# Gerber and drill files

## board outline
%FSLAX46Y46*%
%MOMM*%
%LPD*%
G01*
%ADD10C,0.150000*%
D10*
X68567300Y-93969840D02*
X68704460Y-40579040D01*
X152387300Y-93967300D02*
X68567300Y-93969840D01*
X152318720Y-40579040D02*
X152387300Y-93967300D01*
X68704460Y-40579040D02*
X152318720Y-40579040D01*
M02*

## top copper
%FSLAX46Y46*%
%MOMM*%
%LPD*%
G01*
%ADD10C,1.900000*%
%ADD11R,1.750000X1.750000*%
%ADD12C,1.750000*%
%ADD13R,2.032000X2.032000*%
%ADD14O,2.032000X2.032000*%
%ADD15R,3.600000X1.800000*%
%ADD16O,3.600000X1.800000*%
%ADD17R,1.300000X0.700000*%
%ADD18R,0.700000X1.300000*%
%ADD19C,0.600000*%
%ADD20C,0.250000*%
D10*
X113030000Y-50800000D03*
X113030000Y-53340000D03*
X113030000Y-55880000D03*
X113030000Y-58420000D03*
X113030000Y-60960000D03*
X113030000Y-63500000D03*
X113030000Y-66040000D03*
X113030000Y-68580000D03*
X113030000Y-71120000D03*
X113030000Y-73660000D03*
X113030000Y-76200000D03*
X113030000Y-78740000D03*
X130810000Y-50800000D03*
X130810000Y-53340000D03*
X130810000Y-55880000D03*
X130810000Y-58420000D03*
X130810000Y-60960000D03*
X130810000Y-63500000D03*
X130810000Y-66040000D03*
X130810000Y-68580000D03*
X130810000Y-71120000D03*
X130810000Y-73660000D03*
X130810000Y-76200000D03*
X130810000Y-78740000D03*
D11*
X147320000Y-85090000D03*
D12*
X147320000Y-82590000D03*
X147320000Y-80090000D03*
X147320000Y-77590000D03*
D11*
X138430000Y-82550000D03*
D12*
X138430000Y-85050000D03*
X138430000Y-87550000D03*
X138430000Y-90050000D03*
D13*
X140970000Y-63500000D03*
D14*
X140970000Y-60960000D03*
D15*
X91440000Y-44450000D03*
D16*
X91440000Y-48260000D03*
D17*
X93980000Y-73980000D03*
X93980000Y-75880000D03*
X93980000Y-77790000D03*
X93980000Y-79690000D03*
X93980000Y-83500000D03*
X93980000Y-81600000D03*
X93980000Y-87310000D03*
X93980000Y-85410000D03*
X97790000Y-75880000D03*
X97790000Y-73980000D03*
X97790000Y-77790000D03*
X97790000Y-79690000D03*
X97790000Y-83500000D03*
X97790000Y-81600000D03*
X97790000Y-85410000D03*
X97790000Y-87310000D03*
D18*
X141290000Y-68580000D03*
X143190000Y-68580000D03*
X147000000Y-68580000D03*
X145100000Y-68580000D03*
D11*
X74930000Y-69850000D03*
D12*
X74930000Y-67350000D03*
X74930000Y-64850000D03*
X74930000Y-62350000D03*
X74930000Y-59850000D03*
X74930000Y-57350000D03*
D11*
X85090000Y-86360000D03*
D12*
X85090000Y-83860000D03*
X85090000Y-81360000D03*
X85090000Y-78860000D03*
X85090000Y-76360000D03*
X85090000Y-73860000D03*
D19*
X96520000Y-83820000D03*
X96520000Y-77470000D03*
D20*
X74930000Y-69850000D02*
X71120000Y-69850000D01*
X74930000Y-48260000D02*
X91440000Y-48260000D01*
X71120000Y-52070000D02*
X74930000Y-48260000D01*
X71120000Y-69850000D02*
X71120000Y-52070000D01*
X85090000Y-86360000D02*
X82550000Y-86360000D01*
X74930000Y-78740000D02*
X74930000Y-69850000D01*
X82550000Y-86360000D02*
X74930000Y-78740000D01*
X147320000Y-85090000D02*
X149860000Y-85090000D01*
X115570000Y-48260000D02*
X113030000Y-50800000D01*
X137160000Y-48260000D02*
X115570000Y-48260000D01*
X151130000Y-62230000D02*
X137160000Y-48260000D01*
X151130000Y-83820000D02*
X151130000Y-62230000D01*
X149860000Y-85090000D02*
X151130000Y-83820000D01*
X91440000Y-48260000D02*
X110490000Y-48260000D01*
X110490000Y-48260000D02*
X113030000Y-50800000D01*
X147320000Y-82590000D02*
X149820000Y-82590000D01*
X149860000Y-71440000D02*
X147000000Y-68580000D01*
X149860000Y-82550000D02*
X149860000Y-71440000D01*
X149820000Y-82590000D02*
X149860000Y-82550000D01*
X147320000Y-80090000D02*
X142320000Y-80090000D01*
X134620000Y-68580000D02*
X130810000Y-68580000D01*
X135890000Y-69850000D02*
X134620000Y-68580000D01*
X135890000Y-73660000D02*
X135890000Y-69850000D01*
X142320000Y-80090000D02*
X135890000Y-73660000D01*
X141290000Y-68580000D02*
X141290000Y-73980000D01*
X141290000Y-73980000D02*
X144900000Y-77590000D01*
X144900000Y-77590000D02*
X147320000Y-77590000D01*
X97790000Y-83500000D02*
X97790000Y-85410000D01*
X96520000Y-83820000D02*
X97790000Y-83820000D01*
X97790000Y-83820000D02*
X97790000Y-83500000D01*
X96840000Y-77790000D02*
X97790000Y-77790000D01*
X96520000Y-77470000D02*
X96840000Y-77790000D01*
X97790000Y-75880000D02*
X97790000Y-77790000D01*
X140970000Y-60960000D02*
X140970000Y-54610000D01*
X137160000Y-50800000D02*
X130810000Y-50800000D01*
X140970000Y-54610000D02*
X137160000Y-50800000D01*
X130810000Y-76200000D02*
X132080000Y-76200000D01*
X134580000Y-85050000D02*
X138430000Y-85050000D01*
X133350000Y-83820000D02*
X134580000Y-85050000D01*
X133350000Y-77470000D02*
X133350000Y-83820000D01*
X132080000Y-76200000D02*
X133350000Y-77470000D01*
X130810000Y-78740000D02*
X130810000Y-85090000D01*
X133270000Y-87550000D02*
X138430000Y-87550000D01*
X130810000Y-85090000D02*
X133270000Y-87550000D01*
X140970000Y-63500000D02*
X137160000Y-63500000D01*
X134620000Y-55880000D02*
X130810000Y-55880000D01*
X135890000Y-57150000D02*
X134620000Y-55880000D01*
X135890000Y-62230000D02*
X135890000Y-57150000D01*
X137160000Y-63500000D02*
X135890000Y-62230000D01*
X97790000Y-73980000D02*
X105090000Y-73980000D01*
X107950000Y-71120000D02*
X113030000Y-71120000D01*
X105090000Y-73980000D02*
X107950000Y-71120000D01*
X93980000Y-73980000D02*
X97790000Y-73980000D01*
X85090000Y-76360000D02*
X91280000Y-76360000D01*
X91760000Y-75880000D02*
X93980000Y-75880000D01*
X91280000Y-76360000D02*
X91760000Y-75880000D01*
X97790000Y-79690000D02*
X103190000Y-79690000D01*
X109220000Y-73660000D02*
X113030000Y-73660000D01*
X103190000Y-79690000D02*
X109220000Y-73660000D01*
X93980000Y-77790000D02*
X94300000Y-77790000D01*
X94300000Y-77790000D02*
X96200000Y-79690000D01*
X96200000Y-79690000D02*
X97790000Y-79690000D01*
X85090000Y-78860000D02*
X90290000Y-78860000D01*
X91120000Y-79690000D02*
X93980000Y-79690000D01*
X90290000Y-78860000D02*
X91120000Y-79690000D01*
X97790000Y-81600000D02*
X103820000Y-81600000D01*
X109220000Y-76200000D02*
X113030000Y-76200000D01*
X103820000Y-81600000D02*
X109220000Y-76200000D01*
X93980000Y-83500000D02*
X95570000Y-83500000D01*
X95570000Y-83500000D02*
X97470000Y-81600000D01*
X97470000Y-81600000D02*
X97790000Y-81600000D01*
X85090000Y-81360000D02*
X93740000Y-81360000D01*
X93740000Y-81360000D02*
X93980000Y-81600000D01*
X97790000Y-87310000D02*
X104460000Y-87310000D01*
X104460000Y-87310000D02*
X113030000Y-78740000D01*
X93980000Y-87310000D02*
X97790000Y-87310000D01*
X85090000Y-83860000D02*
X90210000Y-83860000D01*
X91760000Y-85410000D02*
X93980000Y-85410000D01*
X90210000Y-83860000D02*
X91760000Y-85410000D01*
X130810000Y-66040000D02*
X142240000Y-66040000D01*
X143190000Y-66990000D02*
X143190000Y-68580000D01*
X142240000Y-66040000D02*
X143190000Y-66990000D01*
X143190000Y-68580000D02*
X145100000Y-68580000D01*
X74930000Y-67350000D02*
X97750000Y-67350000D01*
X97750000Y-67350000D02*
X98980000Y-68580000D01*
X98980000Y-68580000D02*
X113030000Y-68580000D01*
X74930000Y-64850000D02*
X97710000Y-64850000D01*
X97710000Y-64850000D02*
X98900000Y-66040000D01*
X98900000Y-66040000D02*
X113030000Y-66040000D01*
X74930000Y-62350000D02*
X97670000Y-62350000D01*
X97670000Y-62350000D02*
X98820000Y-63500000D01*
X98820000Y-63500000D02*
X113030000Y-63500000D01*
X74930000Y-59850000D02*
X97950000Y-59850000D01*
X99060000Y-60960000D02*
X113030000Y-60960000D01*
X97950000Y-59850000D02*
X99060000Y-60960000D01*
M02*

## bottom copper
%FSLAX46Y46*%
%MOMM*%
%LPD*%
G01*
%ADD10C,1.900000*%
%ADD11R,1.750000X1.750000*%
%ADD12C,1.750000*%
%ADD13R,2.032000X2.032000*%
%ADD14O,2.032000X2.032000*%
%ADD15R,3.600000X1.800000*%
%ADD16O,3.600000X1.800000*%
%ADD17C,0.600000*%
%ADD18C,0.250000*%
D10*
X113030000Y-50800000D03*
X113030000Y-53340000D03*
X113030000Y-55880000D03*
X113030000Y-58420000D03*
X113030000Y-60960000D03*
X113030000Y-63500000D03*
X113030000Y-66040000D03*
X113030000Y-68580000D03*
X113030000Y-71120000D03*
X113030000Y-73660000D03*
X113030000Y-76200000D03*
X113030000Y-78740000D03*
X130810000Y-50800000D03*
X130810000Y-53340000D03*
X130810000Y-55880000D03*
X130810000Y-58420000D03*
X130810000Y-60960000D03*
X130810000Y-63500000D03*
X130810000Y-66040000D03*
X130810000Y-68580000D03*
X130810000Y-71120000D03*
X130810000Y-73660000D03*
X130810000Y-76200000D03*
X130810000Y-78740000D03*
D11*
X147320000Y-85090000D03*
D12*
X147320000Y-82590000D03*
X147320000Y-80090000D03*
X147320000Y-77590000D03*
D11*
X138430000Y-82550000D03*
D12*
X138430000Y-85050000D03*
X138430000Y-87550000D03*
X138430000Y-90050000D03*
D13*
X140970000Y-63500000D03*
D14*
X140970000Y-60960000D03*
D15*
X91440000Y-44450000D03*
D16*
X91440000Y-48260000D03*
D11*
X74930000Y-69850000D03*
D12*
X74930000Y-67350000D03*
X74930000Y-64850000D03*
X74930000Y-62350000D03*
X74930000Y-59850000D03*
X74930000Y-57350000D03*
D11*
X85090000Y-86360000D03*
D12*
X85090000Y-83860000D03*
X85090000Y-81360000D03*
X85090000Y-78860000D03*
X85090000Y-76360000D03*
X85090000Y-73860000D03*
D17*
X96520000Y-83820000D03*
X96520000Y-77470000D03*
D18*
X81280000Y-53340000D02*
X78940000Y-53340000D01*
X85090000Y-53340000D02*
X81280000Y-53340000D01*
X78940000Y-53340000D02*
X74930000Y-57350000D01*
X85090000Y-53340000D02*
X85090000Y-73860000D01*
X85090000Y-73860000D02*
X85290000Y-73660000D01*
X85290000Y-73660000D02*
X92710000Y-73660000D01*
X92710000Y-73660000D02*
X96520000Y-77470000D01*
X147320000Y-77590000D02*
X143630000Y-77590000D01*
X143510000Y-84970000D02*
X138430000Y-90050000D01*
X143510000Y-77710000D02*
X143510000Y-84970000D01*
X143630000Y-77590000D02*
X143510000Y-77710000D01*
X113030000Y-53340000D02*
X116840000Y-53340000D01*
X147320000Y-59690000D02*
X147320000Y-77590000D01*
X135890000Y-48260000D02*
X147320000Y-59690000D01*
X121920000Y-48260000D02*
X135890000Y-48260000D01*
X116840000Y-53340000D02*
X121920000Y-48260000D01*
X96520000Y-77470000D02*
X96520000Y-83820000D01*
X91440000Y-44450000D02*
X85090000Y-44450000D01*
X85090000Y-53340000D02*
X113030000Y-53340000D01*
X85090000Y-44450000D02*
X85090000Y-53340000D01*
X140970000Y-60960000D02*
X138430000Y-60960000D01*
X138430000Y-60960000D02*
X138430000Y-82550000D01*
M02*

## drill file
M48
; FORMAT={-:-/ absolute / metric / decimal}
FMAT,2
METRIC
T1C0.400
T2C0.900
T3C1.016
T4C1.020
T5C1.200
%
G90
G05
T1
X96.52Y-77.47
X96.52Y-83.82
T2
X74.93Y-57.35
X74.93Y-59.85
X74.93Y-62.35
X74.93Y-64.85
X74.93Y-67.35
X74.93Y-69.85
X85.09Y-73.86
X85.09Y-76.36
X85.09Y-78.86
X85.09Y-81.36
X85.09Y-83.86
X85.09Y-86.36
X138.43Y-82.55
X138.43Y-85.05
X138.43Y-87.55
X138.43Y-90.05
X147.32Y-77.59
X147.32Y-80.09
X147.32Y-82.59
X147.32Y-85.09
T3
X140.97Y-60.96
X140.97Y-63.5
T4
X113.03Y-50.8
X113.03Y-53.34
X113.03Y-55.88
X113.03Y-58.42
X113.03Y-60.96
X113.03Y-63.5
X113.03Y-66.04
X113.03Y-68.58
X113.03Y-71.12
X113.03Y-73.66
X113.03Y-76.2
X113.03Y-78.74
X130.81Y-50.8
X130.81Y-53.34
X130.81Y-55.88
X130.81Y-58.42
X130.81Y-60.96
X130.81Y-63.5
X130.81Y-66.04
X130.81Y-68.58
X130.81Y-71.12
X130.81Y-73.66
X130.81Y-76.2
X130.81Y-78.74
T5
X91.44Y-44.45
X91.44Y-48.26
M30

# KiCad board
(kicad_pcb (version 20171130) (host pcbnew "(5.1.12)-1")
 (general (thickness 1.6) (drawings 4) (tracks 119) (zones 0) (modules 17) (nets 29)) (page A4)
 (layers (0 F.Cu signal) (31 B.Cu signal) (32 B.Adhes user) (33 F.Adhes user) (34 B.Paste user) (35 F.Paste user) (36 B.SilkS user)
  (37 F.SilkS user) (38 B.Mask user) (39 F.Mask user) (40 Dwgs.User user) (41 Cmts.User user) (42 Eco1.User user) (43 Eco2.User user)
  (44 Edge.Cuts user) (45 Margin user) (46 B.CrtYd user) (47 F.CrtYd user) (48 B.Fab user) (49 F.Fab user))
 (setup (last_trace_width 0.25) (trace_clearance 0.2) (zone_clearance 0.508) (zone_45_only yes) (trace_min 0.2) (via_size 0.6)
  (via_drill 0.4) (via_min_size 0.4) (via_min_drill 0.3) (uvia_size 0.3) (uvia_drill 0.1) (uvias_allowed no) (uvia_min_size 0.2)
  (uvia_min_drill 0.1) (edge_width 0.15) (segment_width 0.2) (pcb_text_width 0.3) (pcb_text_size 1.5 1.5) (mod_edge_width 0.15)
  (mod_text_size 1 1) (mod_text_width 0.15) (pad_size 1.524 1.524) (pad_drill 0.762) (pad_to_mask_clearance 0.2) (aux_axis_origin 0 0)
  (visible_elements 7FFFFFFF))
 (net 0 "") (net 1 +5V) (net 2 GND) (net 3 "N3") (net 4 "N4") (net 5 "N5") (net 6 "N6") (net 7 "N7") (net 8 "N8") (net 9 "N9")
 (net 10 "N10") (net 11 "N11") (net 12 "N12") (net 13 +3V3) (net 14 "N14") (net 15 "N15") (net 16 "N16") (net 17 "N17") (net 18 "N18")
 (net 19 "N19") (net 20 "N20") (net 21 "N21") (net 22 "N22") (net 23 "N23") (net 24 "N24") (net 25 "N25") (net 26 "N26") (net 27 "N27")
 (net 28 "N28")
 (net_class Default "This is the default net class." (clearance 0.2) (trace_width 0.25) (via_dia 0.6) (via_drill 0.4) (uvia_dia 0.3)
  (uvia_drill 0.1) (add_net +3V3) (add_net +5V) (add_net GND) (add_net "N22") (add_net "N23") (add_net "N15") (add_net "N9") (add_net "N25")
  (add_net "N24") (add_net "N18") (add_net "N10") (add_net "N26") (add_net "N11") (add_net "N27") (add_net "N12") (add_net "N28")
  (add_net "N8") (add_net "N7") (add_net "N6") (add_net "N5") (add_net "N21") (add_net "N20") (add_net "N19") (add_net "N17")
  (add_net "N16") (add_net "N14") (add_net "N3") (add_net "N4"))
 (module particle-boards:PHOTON (layer F.Cu) (at 121.92 66.04)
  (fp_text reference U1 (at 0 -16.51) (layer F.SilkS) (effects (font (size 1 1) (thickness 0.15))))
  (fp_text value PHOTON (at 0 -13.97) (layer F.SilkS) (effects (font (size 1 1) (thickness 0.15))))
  (pad 1 thru_hole circle (at -8.89 -15.24) (size 1.9 1.9) (drill 1.02) (layers *.Cu *.Mask F.SilkS) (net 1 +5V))
  (pad 2 thru_hole circle (at -8.89 -12.7) (size 1.9 1.9) (drill 1.02) (layers *.Cu *.Mask F.SilkS) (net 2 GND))
  (pad 3 thru_hole circle (at -8.89 -10.16) (size 1.9 1.9) (drill 1.02) (layers *.Cu *.Mask F.SilkS) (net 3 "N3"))
  (pad 4 thru_hole circle (at -8.89 -7.62) (size 1.9 1.9) (drill 1.02) (layers *.Cu *.Mask F.SilkS) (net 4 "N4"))
  (pad 5 thru_hole circle (at -8.89 -5.08) (size 1.9 1.9) (drill 1.02) (layers *.Cu *.Mask F.SilkS) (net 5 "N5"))
  (pad 6 thru_hole circle (at -8.89 -2.54) (size 1.9 1.9) (drill 1.02) (layers *.Cu *.Mask F.SilkS) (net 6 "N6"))
  (pad 7 thru_hole circle (at -8.89 0) (size 1.9 1.9) (drill 1.02) (layers *.Cu *.Mask F.SilkS) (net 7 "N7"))
  (pad 8 thru_hole circle (at -8.89 2.54) (size 1.9 1.9) (drill 1.02) (layers *.Cu *.Mask F.SilkS) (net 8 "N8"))
  (pad 9 thru_hole circle (at -8.89 5.08) (size 1.9 1.9) (drill 1.02) (layers *.Cu *.Mask F.SilkS) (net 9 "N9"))
  (pad 10 thru_hole circle (at -8.89 7.62) (size 1.9 1.9) (drill 1.02) (layers *.Cu *.Mask F.SilkS) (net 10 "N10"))
  (pad 11 thru_hole circle (at -8.89 10.16) (size 1.9 1.9) (drill 1.02) (layers *.Cu *.Mask F.SilkS) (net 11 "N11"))
  (pad 12 thru_hole circle (at -8.89 12.7) (size 1.9 1.9) (drill 1.02) (layers *.Cu *.Mask F.SilkS) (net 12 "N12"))
  (pad 24 thru_hole circle (at 8.89 -15.24) (size 1.9 1.9) (drill 1.02) (layers *.Cu *.Mask F.SilkS) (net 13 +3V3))
  (pad 23 thru_hole circle (at 8.89 -12.7) (size 1.9 1.9) (drill 1.02) (layers *.Cu *.Mask F.SilkS) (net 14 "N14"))
  (pad 22 thru_hole circle (at 8.89 -10.16) (size 1.9 1.9) (drill 1.02) (layers *.Cu *.Mask F.SilkS) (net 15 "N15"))
  (pad 21 thru_hole circle (at 8.89 -7.62) (size 1.9 1.9) (drill 1.02) (layers *.Cu *.Mask F.SilkS))
  (pad 20 thru_hole circle (at 8.89 -5.08) (size 1.9 1.9) (drill 1.02) (layers *.Cu *.Mask F.SilkS) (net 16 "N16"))
  (pad 19 thru_hole circle (at 8.89 -2.54) (size 1.9 1.9) (drill 1.02) (layers *.Cu *.Mask F.SilkS) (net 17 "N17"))
  (pad 18 thru_hole circle (at 8.89 0) (size 1.9 1.9) (drill 1.02) (layers *.Cu *.Mask F.SilkS) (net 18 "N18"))
  (pad 17 thru_hole circle (at 8.89 2.54) (size 1.9 1.9) (drill 1.02) (layers *.Cu *.Mask F.SilkS) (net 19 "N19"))
  (pad 16 thru_hole circle (at 8.89 5.08) (size 1.9 1.9) (drill 1.02) (layers *.Cu *.Mask F.SilkS) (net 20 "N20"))
  (pad 15 thru_hole circle (at 8.89 7.62) (size 1.9 1.9) (drill 1.02) (layers *.Cu *.Mask F.SilkS) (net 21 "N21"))
  (pad 14 thru_hole circle (at 8.89 10.16) (size 1.9 1.9) (drill 1.02) (layers *.Cu *.Mask F.SilkS) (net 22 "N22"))
  (pad 13 thru_hole circle (at 8.89 12.7) (size 1.9 1.9) (drill 1.02) (layers *.Cu *.Mask F.SilkS) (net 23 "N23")))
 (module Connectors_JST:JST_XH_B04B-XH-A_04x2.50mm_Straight (layer F.Cu) (at 147.32 85.09 90)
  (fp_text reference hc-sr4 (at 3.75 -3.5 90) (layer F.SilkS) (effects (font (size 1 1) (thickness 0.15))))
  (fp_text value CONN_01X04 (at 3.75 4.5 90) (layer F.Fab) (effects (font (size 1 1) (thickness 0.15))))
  (pad 1 thru_hole rect (at 0 0 90) (size 1.75 1.75) (drill 0.9) (layers *.Cu *.Mask) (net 1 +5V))
  (pad 2 thru_hole circle (at 2.5 0 90) (size 1.75 1.75) (drill 0.9) (layers *.Cu *.Mask) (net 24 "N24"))
  (pad 3 thru_hole circle (at 5 0 90) (size 1.75 1.75) (drill 0.9) (layers *.Cu *.Mask) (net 19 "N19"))
  (pad 4 thru_hole circle (at 7.5 0 90) (size 1.75 1.75) (drill 0.9) (layers *.Cu *.Mask) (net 2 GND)))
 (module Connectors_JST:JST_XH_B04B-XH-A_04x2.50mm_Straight (layer F.Cu) (at 138.43 82.55 270)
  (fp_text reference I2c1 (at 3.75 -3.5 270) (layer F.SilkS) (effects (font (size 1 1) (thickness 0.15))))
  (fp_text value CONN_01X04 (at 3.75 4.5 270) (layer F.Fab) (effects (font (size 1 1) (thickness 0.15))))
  (pad 1 thru_hole rect (at 0 0 270) (size 1.75 1.75) (drill 0.9) (layers *.Cu *.Mask) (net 13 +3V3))
  (pad 2 thru_hole circle (at 2.5 0 270) (size 1.75 1.75) (drill 0.9) (layers *.Cu *.Mask) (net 22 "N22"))
  (pad 3 thru_hole circle (at 5 0 270) (size 1.75 1.75) (drill 0.9) (layers *.Cu *.Mask) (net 23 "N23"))
  (pad 4 thru_hole circle (at 7.5 0 270) (size 1.75 1.75) (drill 0.9) (layers *.Cu *.Mask) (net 2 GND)))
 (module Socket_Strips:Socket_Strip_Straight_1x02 (layer F.Cu) (at 140.97 63.5 90)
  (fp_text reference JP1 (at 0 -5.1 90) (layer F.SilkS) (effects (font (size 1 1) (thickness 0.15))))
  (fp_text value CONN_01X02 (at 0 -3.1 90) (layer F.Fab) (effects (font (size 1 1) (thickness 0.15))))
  (pad 1 thru_hole rect (at 0 0 90) (size 2.032 2.032) (drill 1.016) (layers *.Cu *.Mask F.SilkS) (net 15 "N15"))
  (pad 2 thru_hole oval (at 2.54 0 90) (size 2.032 2.032) (drill 1.016) (layers *.Cu *.Mask F.SilkS) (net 13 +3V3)))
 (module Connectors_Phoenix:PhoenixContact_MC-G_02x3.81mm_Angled (layer F.Cu) (at 91.44 44.45 270)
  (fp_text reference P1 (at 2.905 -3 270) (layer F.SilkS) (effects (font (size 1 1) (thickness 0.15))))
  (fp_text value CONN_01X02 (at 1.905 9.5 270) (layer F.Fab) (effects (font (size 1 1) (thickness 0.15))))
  (pad 1 thru_hole rect (at 0 0 270) (size 1.8 3.6) (drill 1.2) (layers *.Cu *.Mask) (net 2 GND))
  (pad 2 thru_hole oval (at 3.81 0 270) (size 1.8 3.6) (drill 1.2) (layers *.Cu *.Mask) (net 1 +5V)))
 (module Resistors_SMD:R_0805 (layer F.Cu) (at 93.98 74.93 270)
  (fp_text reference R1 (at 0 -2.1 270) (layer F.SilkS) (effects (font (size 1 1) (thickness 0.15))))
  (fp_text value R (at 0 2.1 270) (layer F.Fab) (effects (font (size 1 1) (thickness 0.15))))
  (pad 1 smd rect (at -0.95 0 270) (size 0.7 1.3) (layers F.Cu F.Paste F.Mask) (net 9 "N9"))
  (pad 2 smd rect (at 0.95 0 270) (size 0.7 1.3) (layers F.Cu F.Paste F.Mask) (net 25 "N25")))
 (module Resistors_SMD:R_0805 (layer F.Cu) (at 93.98 78.74 270)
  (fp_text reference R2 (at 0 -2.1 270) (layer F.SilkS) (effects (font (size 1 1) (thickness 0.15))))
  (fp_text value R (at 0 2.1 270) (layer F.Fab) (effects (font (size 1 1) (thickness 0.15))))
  (pad 1 smd rect (at -0.95 0 270) (size 0.7 1.3) (layers F.Cu F.Paste F.Mask) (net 10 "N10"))
  (pad 2 smd rect (at 0.95 0 270) (size 0.7 1.3) (layers F.Cu F.Paste F.Mask) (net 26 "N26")))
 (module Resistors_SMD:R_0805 (layer F.Cu) (at 93.98 82.55 90)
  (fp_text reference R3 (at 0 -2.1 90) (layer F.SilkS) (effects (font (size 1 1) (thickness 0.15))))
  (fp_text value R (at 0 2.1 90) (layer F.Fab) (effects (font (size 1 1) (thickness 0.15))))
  (pad 1 smd rect (at -0.95 0 90) (size 0.7 1.3) (layers F.Cu F.Paste F.Mask) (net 11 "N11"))
  (pad 2 smd rect (at 0.95 0 90) (size 0.7 1.3) (layers F.Cu F.Paste F.Mask) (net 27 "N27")))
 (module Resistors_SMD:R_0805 (layer F.Cu) (at 93.98 86.36 90)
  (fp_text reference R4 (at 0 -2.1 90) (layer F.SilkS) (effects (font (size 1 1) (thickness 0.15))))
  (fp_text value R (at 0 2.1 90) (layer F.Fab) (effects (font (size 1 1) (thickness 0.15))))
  (pad 1 smd rect (at -0.95 0 90) (size 0.7 1.3) (layers F.Cu F.Paste F.Mask) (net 12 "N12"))
  (pad 2 smd rect (at 0.95 0 90) (size 0.7 1.3) (layers F.Cu F.Paste F.Mask) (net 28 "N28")))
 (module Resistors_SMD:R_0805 (layer F.Cu) (at 97.79 74.93 90)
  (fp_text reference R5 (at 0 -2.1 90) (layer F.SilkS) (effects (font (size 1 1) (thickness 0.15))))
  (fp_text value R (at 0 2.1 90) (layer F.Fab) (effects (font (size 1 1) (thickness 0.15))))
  (pad 1 smd rect (at -0.95 0 90) (size 0.7 1.3) (layers F.Cu F.Paste F.Mask) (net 2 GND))
  (pad 2 smd rect (at 0.95 0 90) (size 0.7 1.3) (layers F.Cu F.Paste F.Mask) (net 9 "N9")))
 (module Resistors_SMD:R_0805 (layer F.Cu) (at 97.79 78.74 270)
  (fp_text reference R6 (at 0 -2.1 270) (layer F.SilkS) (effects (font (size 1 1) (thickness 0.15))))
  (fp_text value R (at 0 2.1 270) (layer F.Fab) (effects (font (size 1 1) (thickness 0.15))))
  (pad 1 smd rect (at -0.95 0 270) (size 0.7 1.3) (layers F.Cu F.Paste F.Mask) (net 2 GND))
  (pad 2 smd rect (at 0.95 0 270) (size 0.7 1.3) (layers F.Cu F.Paste F.Mask) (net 10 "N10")))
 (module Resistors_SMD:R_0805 (layer F.Cu) (at 97.79 82.55 90)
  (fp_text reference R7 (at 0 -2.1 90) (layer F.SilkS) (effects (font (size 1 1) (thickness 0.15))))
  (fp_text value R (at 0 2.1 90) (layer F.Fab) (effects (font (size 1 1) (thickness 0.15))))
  (pad 1 smd rect (at -0.95 0 90) (size 0.7 1.3) (layers F.Cu F.Paste F.Mask) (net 2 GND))
  (pad 2 smd rect (at 0.95 0 90) (size 0.7 1.3) (layers F.Cu F.Paste F.Mask) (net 11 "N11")))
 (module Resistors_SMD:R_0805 (layer F.Cu) (at 97.79 86.36 270)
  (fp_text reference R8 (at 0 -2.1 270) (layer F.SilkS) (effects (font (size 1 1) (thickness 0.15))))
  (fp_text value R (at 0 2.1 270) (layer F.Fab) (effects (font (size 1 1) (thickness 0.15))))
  (pad 1 smd rect (at -0.95 0 270) (size 0.7 1.3) (layers F.Cu F.Paste F.Mask) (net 2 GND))
  (pad 2 smd rect (at 0.95 0 270) (size 0.7 1.3) (layers F.Cu F.Paste F.Mask) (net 12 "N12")))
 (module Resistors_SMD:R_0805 (layer F.Cu) (at 142.24 68.58)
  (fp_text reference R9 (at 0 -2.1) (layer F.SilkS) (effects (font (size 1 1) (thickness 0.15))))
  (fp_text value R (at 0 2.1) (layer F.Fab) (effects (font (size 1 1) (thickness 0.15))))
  (pad 1 smd rect (at -0.95 0) (size 0.7 1.3) (layers F.Cu F.Paste F.Mask) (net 2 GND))
  (pad 2 smd rect (at 0.95 0) (size 0.7 1.3) (layers F.Cu F.Paste F.Mask) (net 18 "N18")))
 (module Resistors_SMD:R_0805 (layer F.Cu) (at 146.05 68.58 180)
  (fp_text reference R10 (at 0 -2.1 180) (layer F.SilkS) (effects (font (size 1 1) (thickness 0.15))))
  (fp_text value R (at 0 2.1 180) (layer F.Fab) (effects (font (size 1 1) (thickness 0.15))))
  (pad 1 smd rect (at -0.95 0 180) (size 0.7 1.3) (layers F.Cu F.Paste F.Mask) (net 24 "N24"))
  (pad 2 smd rect (at 0.95 0 180) (size 0.7 1.3) (layers F.Cu F.Paste F.Mask) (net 18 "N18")))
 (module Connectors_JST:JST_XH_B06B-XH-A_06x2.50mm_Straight (layer F.Cu) (at 74.93 69.85 90)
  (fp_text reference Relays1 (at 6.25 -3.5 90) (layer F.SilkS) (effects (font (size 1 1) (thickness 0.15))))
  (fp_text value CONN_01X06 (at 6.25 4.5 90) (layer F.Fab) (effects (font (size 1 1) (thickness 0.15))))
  (pad 1 thru_hole rect (at 0 0 90) (size 1.75 1.75) (drill 0.9) (layers *.Cu *.Mask) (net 1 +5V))
  (pad 2 thru_hole circle (at 2.5 0 90) (size 1.75 1.75) (drill 0.9) (layers *.Cu *.Mask) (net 8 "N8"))
  (pad 3 thru_hole circle (at 5 0 90) (size 1.75 1.75) (drill 0.9) (layers *.Cu *.Mask) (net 7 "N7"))
  (pad 4 thru_hole circle (at 7.5 0 90) (size 1.75 1.75) (drill 0.9) (layers *.Cu *.Mask) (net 6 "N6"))
  (pad 5 thru_hole circle (at 10 0 90) (size 1.75 1.75) (drill 0.9) (layers *.Cu *.Mask) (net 5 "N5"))
  (pad 6 thru_hole circle (at 12.5 0 90) (size 1.75 1.75) (drill 0.9) (layers *.Cu *.Mask) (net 2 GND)))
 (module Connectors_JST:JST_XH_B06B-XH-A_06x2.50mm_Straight (layer F.Cu) (at 85.09 86.36 90)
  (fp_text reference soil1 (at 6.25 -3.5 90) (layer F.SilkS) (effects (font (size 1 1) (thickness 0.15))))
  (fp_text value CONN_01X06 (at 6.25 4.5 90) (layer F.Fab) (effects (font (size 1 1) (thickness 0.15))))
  (pad 1 thru_hole rect (at 0 0 90) (size 1.75 1.75) (drill 0.9) (layers *.Cu *.Mask) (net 1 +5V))
  (pad 2 thru_hole circle (at 2.5 0 90) (size 1.75 1.75) (drill 0.9) (layers *.Cu *.Mask) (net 28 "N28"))
  (pad 3 thru_hole circle (at 5 0 90) (size 1.75 1.75) (drill 0.9) (layers *.Cu *.Mask) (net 27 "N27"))
  (pad 4 thru_hole circle (at 7.5 0 90) (size 1.75 1.75) (drill 0.9) (layers *.Cu *.Mask) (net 26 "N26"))
  (pad 5 thru_hole circle (at 10 0 90) (size 1.75 1.75) (drill 0.9) (layers *.Cu *.Mask) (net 25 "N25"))
  (pad 6 thru_hole circle (at 12.5 0 90) (size 1.75 1.75) (drill 0.9) (layers *.Cu *.Mask) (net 2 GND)))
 (gr_line (start 68.5673 93.96984) (end 68.70446 40.57904) (layer Edge.Cuts) (width 0.15))
 (gr_line (start 152.3873 93.9673) (end 68.5673 93.96984) (layer Edge.Cuts) (width 0.15))
 (gr_line (start 152.31872 40.57904) (end 152.3873 93.9673) (layer Edge.Cuts) (width 0.15))
 (gr_line (start 68.70446 40.57904) (end 152.31872 40.57904) (layer Edge.Cuts) (width 0.15))
 (segment (start 74.93 69.85) (end 71.12 69.85) (width 0.25) (layer F.Cu) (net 1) (status 400000))
 (segment (start 74.93 48.26) (end 91.44 48.26) (width 0.25) (layer F.Cu) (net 1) (status 800000))
 (segment (start 71.12 52.07) (end 74.93 48.26) (width 0.25) (layer F.Cu) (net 1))
 (segment (start 71.12 69.85) (end 71.12 52.07) (width 0.25) (layer F.Cu) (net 1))
 (segment (start 85.09 86.36) (end 82.55 86.36) (width 0.25) (layer F.Cu) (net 1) (status 400000))
 (segment (start 74.93 78.74) (end 74.93 69.85) (width 0.25) (layer F.Cu) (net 1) (status 800000))
 (segment (start 82.55 86.36) (end 74.93 78.74) (width 0.25) (layer F.Cu) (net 1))
 (segment (start 147.32 85.09) (end 149.86 85.09) (width 0.25) (layer F.Cu) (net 1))
 (segment (start 115.57 48.26) (end 113.03 50.8) (width 0.25) (layer F.Cu) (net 1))
 (segment (start 137.16 48.26) (end 115.57 48.26) (width 0.25) (layer F.Cu) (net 1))
 (segment (start 151.13 62.23) (end 137.16 48.26) (width 0.25) (layer F.Cu) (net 1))
 (segment (start 151.13 83.82) (end 151.13 62.23) (width 0.25) (layer F.Cu) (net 1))
 (segment (start 149.86 85.09) (end 151.13 83.82) (width 0.25) (layer F.Cu) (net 1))
 (segment (start 91.44 48.26) (end 110.49 48.26) (width 0.25) (layer F.Cu) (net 1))
 (segment (start 110.49 48.26) (end 113.03 50.8) (width 0.25) (layer F.Cu) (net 1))
 (segment (start 147.32 82.59) (end 149.82 82.59) (width 0.25) (layer F.Cu) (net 24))
 (segment (start 149.86 71.44) (end 147 68.58) (width 0.25) (layer F.Cu) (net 24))
 (segment (start 149.86 82.55) (end 149.86 71.44) (width 0.25) (layer F.Cu) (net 24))
 (segment (start 149.82 82.59) (end 149.86 82.55) (width 0.25) (layer F.Cu) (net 24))
 (segment (start 147.32 80.09) (end 142.32 80.09) (width 0.25) (layer F.Cu) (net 19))
 (segment (start 134.62 68.58) (end 130.81 68.58) (width 0.25) (layer F.Cu) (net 19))
 (segment (start 135.89 69.85) (end 134.62 68.58) (width 0.25) (layer F.Cu) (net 19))
 (segment (start 135.89 73.66) (end 135.89 69.85) (width 0.25) (layer F.Cu) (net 19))
 (segment (start 142.32 80.09) (end 135.89 73.66) (width 0.25) (layer F.Cu) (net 19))
 (segment (start 81.28 53.34) (end 78.94 53.34) (width 0.25) (layer B.Cu) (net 2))
 (segment (start 85.09 53.34) (end 81.28 53.34) (width 0.25) (layer B.Cu) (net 2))
 (segment (start 78.94 53.34) (end 74.93 57.35) (width 0.25) (layer B.Cu) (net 2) (status 800000))
 (segment (start 85.09 53.34) (end 85.09 73.86) (width 0.25) (layer B.Cu) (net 2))
 (segment (start 85.09 73.86) (end 85.29 73.66) (width 0.25) (layer B.Cu) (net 2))
 (segment (start 85.29 73.66) (end 92.71 73.66) (width 0.25) (layer B.Cu) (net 2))
 (segment (start 92.71 73.66) (end 96.52 77.47) (width 0.25) (layer B.Cu) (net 2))
 (segment (start 147.32 77.59) (end 143.63 77.59) (width 0.25) (layer B.Cu) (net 2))
 (segment (start 143.51 84.97) (end 138.43 90.05) (width 0.25) (layer B.Cu) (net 2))
 (segment (start 143.51 77.71) (end 143.51 84.97) (width 0.25) (layer B.Cu) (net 2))
 (segment (start 143.63 77.59) (end 143.51 77.71) (width 0.25) (layer B.Cu) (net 2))
 (segment (start 113.03 53.34) (end 116.84 53.34) (width 0.25) (layer B.Cu) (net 2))
 (segment (start 147.32 59.69) (end 147.32 77.59) (width 0.25) (layer B.Cu) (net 2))
 (segment (start 135.89 48.26) (end 147.32 59.69) (width 0.25) (layer B.Cu) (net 2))
 (segment (start 121.92 48.26) (end 135.89 48.26) (width 0.25) (layer B.Cu) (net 2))
 (segment (start 116.84 53.34) (end 121.92 48.26) (width 0.25) (layer B.Cu) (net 2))
 (segment (start 141.29 68.58) (end 141.29 73.98) (width 0.25) (layer F.Cu) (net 2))
 (segment (start 141.29 73.98) (end 144.9 77.59) (width 0.25) (layer F.Cu) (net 2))
 (segment (start 144.9 77.59) (end 147.32 77.59) (width 0.25) (layer F.Cu) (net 2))
 (segment (start 97.79 83.5) (end 97.79 85.41) (width 0.25) (layer F.Cu) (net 2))
 (segment (start 96.52 77.47) (end 96.52 83.82) (width 0.25) (layer B.Cu) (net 2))
 (segment (start 96.52 83.82) (end 97.79 83.82) (width 0.25) (layer F.Cu) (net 2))
 (via (at 96.52 83.82) (size 0.6) (drill 0.4) (layers F.Cu B.Cu) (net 2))
 (segment (start 97.79 83.82) (end 97.79 83.5) (width 0.25) (layer F.Cu) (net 2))
 (segment (start 96.84 77.79) (end 97.79 77.79) (width 0.25) (layer F.Cu) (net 2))
 (segment (start 96.52 77.47) (end 96.84 77.79) (width 0.25) (layer F.Cu) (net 2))
 (via (at 96.52 77.47) (size 0.6) (drill 0.4) (layers F.Cu B.Cu) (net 2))
 (segment (start 97.79 75.88) (end 97.79 77.79) (width 0.25) (layer F.Cu) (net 2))
 (segment (start 91.44 44.45) (end 85.09 44.45) (width 0.25) (layer B.Cu) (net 2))
 (segment (start 85.09 53.34) (end 113.03 53.34) (width 0.25) (layer B.Cu) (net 2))
 (segment (start 85.09 44.45) (end 85.09 53.34) (width 0.25) (layer B.Cu) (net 2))
 (segment (start 140.97 60.96) (end 138.43 60.96) (width 0.25) (layer B.Cu) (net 13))
 (segment (start 138.43 60.96) (end 138.43 82.55) (width 0.25) (layer B.Cu) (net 13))
 (segment (start 140.97 60.96) (end 140.97 54.61) (width 0.25) (layer F.Cu) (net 13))
 (segment (start 137.16 50.8) (end 130.81 50.8) (width 0.25) (layer F.Cu) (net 13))
 (segment (start 140.97 54.61) (end 137.16 50.8) (width 0.25) (layer F.Cu) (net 13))
 (segment (start 130.81 76.2) (end 132.08 76.2) (width 0.25) (layer F.Cu) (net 22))
 (segment (start 134.58 85.05) (end 138.43 85.05) (width 0.25) (layer F.Cu) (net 22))
 (segment (start 133.35 83.82) (end 134.58 85.05) (width 0.25) (layer F.Cu) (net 22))
 (segment (start 133.35 77.47) (end 133.35 83.82) (width 0.25) (layer F.Cu) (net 22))
 (segment (start 132.08 76.2) (end 133.35 77.47) (width 0.25) (layer F.Cu) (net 22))
 (segment (start 130.81 78.74) (end 130.81 85.09) (width 0.25) (layer F.Cu) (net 23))
 (segment (start 133.27 87.55) (end 138.43 87.55) (width 0.25) (layer F.Cu) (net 23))
 (segment (start 130.81 85.09) (end 133.27 87.55) (width 0.25) (layer F.Cu) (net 23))
 (segment (start 140.97 63.5) (end 137.16 63.5) (width 0.25) (layer F.Cu) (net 15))
 (segment (start 134.62 55.88) (end 130.81 55.88) (width 0.25) (layer F.Cu) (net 15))
 (segment (start 135.89 57.15) (end 134.62 55.88) (width 0.25) (layer F.Cu) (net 15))
 (segment (start 135.89 62.23) (end 135.89 57.15) (width 0.25) (layer F.Cu) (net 15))
 (segment (start 137.16 63.5) (end 135.89 62.23) (width 0.25) (layer F.Cu) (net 15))
 (segment (start 97.79 73.98) (end 105.09 73.98) (width 0.25) (layer F.Cu) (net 9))
 (segment (start 107.95 71.12) (end 113.03 71.12) (width 0.25) (layer F.Cu) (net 9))
 (segment (start 105.09 73.98) (end 107.95 71.12) (width 0.25) (layer F.Cu) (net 9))
 (segment (start 93.98 73.98) (end 97.79 73.98) (width 0.25) (layer F.Cu) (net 9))
 (segment (start 85.09 76.36) (end 91.28 76.36) (width 0.25) (layer F.Cu) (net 25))
 (segment (start 91.76 75.88) (end 93.98 75.88) (width 0.25) (layer F.Cu) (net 25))
 (segment (start 91.28 76.36) (end 91.76 75.88) (width 0.25) (layer F.Cu) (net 25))
 (segment (start 97.79 79.69) (end 103.19 79.69) (width 0.25) (layer F.Cu) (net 10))
 (segment (start 109.22 73.66) (end 113.03 73.66) (width 0.25) (layer F.Cu) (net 10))
 (segment (start 103.19 79.69) (end 109.22 73.66) (width 0.25) (layer F.Cu) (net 10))
 (segment (start 93.98 77.79) (end 94.3 77.79) (width 0.25) (layer F.Cu) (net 10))
 (segment (start 94.3 77.79) (end 96.2 79.69) (width 0.25) (layer F.Cu) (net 10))
 (segment (start 96.2 79.69) (end 97.79 79.69) (width 0.25) (layer F.Cu) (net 10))
 (segment (start 85.09 78.86) (end 90.29 78.86) (width 0.25) (layer F.Cu) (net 26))
 (segment (start 91.12 79.69) (end 93.98 79.69) (width 0.25) (layer F.Cu) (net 26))
 (segment (start 90.29 78.86) (end 91.12 79.69) (width 0.25) (layer F.Cu) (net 26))
 (segment (start 97.79 81.6) (end 103.82 81.6) (width 0.25) (layer F.Cu) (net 11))
 (segment (start 109.22 76.2) (end 113.03 76.2) (width 0.25) (layer F.Cu) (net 11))
 (segment (start 103.82 81.6) (end 109.22 76.2) (width 0.25) (layer F.Cu) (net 11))
 (segment (start 93.98 83.5) (end 95.57 83.5) (width 0.25) (layer F.Cu) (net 11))
 (segment (start 95.57 83.5) (end 97.47 81.6) (width 0.25) (layer F.Cu) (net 11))
 (segment (start 97.47 81.6) (end 97.79 81.6) (width 0.25) (layer F.Cu) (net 11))
 (segment (start 85.09 81.36) (end 93.74 81.36) (width 0.25) (layer F.Cu) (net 27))
 (segment (start 93.74 81.36) (end 93.98 81.6) (width 0.25) (layer F.Cu) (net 27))
 (segment (start 97.79 87.31) (end 104.46 87.31) (width 0.25) (layer F.Cu) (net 12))
 (segment (start 104.46 87.31) (end 113.03 78.74) (width 0.25) (layer F.Cu) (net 12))
 (segment (start 93.98 87.31) (end 97.79 87.31) (width 0.25) (layer F.Cu) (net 12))
 (segment (start 85.09 83.86) (end 90.21 83.86) (width 0.25) (layer F.Cu) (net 28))
 (segment (start 91.76 85.41) (end 93.98 85.41) (width 0.25) (layer F.Cu) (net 28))
 (segment (start 90.21 83.86) (end 91.76 85.41) (width 0.25) (layer F.Cu) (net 28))
 (segment (start 130.81 66.04) (end 142.24 66.04) (width 0.25) (layer F.Cu) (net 18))
 (segment (start 143.19 66.99) (end 143.19 68.58) (width 0.25) (layer F.Cu) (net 18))
 (segment (start 142.24 66.04) (end 143.19 66.99) (width 0.25) (layer F.Cu) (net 18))
 (segment (start 143.19 68.58) (end 145.1 68.58) (width 0.25) (layer F.Cu) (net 18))
 (segment (start 74.93 67.35) (end 97.75 67.35) (width 0.25) (layer F.Cu) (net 8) (status 400000))
 (segment (start 97.75 67.35) (end 98.98 68.58) (width 0.25) (layer F.Cu) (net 8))
 (segment (start 98.98 68.58) (end 113.03 68.58) (width 0.25) (layer F.Cu) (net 8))
 (segment (start 74.93 64.85) (end 97.71 64.85) (width 0.25) (layer F.Cu) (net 7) (status 400000))
 (segment (start 97.71 64.85) (end 98.9 66.04) (width 0.25) (layer F.Cu) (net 7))
 (segment (start 98.9 66.04) (end 113.03 66.04) (width 0.25) (layer F.Cu) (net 7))
 (segment (start 74.93 62.35) (end 97.67 62.35) (width 0.25) (layer F.Cu) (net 6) (status 400000))
 (segment (start 97.67 62.35) (end 98.82 63.5) (width 0.25) (layer F.Cu) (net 6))
 (segment (start 98.82 63.5) (end 113.03 63.5) (width 0.25) (layer F.Cu) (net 6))
 (segment (start 74.93 59.85) (end 97.95 59.85) (width 0.25) (layer F.Cu) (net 5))
 (segment (start 99.06 60.96) (end 113.03 60.96) (width 0.25) (layer F.Cu) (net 5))
 (segment (start 97.95 59.85) (end 99.06 60.96) (width 0.25) (layer F.Cu) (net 5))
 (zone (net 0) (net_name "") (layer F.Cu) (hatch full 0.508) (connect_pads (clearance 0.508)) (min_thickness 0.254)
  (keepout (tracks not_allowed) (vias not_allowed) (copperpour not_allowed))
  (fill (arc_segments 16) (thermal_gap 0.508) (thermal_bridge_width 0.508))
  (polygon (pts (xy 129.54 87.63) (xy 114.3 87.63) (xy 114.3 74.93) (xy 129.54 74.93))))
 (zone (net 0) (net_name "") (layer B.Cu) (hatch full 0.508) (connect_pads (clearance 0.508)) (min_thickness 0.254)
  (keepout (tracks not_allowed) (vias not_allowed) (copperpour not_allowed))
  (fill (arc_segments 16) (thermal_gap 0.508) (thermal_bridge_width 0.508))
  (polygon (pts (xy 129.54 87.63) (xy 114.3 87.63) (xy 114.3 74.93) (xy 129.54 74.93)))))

